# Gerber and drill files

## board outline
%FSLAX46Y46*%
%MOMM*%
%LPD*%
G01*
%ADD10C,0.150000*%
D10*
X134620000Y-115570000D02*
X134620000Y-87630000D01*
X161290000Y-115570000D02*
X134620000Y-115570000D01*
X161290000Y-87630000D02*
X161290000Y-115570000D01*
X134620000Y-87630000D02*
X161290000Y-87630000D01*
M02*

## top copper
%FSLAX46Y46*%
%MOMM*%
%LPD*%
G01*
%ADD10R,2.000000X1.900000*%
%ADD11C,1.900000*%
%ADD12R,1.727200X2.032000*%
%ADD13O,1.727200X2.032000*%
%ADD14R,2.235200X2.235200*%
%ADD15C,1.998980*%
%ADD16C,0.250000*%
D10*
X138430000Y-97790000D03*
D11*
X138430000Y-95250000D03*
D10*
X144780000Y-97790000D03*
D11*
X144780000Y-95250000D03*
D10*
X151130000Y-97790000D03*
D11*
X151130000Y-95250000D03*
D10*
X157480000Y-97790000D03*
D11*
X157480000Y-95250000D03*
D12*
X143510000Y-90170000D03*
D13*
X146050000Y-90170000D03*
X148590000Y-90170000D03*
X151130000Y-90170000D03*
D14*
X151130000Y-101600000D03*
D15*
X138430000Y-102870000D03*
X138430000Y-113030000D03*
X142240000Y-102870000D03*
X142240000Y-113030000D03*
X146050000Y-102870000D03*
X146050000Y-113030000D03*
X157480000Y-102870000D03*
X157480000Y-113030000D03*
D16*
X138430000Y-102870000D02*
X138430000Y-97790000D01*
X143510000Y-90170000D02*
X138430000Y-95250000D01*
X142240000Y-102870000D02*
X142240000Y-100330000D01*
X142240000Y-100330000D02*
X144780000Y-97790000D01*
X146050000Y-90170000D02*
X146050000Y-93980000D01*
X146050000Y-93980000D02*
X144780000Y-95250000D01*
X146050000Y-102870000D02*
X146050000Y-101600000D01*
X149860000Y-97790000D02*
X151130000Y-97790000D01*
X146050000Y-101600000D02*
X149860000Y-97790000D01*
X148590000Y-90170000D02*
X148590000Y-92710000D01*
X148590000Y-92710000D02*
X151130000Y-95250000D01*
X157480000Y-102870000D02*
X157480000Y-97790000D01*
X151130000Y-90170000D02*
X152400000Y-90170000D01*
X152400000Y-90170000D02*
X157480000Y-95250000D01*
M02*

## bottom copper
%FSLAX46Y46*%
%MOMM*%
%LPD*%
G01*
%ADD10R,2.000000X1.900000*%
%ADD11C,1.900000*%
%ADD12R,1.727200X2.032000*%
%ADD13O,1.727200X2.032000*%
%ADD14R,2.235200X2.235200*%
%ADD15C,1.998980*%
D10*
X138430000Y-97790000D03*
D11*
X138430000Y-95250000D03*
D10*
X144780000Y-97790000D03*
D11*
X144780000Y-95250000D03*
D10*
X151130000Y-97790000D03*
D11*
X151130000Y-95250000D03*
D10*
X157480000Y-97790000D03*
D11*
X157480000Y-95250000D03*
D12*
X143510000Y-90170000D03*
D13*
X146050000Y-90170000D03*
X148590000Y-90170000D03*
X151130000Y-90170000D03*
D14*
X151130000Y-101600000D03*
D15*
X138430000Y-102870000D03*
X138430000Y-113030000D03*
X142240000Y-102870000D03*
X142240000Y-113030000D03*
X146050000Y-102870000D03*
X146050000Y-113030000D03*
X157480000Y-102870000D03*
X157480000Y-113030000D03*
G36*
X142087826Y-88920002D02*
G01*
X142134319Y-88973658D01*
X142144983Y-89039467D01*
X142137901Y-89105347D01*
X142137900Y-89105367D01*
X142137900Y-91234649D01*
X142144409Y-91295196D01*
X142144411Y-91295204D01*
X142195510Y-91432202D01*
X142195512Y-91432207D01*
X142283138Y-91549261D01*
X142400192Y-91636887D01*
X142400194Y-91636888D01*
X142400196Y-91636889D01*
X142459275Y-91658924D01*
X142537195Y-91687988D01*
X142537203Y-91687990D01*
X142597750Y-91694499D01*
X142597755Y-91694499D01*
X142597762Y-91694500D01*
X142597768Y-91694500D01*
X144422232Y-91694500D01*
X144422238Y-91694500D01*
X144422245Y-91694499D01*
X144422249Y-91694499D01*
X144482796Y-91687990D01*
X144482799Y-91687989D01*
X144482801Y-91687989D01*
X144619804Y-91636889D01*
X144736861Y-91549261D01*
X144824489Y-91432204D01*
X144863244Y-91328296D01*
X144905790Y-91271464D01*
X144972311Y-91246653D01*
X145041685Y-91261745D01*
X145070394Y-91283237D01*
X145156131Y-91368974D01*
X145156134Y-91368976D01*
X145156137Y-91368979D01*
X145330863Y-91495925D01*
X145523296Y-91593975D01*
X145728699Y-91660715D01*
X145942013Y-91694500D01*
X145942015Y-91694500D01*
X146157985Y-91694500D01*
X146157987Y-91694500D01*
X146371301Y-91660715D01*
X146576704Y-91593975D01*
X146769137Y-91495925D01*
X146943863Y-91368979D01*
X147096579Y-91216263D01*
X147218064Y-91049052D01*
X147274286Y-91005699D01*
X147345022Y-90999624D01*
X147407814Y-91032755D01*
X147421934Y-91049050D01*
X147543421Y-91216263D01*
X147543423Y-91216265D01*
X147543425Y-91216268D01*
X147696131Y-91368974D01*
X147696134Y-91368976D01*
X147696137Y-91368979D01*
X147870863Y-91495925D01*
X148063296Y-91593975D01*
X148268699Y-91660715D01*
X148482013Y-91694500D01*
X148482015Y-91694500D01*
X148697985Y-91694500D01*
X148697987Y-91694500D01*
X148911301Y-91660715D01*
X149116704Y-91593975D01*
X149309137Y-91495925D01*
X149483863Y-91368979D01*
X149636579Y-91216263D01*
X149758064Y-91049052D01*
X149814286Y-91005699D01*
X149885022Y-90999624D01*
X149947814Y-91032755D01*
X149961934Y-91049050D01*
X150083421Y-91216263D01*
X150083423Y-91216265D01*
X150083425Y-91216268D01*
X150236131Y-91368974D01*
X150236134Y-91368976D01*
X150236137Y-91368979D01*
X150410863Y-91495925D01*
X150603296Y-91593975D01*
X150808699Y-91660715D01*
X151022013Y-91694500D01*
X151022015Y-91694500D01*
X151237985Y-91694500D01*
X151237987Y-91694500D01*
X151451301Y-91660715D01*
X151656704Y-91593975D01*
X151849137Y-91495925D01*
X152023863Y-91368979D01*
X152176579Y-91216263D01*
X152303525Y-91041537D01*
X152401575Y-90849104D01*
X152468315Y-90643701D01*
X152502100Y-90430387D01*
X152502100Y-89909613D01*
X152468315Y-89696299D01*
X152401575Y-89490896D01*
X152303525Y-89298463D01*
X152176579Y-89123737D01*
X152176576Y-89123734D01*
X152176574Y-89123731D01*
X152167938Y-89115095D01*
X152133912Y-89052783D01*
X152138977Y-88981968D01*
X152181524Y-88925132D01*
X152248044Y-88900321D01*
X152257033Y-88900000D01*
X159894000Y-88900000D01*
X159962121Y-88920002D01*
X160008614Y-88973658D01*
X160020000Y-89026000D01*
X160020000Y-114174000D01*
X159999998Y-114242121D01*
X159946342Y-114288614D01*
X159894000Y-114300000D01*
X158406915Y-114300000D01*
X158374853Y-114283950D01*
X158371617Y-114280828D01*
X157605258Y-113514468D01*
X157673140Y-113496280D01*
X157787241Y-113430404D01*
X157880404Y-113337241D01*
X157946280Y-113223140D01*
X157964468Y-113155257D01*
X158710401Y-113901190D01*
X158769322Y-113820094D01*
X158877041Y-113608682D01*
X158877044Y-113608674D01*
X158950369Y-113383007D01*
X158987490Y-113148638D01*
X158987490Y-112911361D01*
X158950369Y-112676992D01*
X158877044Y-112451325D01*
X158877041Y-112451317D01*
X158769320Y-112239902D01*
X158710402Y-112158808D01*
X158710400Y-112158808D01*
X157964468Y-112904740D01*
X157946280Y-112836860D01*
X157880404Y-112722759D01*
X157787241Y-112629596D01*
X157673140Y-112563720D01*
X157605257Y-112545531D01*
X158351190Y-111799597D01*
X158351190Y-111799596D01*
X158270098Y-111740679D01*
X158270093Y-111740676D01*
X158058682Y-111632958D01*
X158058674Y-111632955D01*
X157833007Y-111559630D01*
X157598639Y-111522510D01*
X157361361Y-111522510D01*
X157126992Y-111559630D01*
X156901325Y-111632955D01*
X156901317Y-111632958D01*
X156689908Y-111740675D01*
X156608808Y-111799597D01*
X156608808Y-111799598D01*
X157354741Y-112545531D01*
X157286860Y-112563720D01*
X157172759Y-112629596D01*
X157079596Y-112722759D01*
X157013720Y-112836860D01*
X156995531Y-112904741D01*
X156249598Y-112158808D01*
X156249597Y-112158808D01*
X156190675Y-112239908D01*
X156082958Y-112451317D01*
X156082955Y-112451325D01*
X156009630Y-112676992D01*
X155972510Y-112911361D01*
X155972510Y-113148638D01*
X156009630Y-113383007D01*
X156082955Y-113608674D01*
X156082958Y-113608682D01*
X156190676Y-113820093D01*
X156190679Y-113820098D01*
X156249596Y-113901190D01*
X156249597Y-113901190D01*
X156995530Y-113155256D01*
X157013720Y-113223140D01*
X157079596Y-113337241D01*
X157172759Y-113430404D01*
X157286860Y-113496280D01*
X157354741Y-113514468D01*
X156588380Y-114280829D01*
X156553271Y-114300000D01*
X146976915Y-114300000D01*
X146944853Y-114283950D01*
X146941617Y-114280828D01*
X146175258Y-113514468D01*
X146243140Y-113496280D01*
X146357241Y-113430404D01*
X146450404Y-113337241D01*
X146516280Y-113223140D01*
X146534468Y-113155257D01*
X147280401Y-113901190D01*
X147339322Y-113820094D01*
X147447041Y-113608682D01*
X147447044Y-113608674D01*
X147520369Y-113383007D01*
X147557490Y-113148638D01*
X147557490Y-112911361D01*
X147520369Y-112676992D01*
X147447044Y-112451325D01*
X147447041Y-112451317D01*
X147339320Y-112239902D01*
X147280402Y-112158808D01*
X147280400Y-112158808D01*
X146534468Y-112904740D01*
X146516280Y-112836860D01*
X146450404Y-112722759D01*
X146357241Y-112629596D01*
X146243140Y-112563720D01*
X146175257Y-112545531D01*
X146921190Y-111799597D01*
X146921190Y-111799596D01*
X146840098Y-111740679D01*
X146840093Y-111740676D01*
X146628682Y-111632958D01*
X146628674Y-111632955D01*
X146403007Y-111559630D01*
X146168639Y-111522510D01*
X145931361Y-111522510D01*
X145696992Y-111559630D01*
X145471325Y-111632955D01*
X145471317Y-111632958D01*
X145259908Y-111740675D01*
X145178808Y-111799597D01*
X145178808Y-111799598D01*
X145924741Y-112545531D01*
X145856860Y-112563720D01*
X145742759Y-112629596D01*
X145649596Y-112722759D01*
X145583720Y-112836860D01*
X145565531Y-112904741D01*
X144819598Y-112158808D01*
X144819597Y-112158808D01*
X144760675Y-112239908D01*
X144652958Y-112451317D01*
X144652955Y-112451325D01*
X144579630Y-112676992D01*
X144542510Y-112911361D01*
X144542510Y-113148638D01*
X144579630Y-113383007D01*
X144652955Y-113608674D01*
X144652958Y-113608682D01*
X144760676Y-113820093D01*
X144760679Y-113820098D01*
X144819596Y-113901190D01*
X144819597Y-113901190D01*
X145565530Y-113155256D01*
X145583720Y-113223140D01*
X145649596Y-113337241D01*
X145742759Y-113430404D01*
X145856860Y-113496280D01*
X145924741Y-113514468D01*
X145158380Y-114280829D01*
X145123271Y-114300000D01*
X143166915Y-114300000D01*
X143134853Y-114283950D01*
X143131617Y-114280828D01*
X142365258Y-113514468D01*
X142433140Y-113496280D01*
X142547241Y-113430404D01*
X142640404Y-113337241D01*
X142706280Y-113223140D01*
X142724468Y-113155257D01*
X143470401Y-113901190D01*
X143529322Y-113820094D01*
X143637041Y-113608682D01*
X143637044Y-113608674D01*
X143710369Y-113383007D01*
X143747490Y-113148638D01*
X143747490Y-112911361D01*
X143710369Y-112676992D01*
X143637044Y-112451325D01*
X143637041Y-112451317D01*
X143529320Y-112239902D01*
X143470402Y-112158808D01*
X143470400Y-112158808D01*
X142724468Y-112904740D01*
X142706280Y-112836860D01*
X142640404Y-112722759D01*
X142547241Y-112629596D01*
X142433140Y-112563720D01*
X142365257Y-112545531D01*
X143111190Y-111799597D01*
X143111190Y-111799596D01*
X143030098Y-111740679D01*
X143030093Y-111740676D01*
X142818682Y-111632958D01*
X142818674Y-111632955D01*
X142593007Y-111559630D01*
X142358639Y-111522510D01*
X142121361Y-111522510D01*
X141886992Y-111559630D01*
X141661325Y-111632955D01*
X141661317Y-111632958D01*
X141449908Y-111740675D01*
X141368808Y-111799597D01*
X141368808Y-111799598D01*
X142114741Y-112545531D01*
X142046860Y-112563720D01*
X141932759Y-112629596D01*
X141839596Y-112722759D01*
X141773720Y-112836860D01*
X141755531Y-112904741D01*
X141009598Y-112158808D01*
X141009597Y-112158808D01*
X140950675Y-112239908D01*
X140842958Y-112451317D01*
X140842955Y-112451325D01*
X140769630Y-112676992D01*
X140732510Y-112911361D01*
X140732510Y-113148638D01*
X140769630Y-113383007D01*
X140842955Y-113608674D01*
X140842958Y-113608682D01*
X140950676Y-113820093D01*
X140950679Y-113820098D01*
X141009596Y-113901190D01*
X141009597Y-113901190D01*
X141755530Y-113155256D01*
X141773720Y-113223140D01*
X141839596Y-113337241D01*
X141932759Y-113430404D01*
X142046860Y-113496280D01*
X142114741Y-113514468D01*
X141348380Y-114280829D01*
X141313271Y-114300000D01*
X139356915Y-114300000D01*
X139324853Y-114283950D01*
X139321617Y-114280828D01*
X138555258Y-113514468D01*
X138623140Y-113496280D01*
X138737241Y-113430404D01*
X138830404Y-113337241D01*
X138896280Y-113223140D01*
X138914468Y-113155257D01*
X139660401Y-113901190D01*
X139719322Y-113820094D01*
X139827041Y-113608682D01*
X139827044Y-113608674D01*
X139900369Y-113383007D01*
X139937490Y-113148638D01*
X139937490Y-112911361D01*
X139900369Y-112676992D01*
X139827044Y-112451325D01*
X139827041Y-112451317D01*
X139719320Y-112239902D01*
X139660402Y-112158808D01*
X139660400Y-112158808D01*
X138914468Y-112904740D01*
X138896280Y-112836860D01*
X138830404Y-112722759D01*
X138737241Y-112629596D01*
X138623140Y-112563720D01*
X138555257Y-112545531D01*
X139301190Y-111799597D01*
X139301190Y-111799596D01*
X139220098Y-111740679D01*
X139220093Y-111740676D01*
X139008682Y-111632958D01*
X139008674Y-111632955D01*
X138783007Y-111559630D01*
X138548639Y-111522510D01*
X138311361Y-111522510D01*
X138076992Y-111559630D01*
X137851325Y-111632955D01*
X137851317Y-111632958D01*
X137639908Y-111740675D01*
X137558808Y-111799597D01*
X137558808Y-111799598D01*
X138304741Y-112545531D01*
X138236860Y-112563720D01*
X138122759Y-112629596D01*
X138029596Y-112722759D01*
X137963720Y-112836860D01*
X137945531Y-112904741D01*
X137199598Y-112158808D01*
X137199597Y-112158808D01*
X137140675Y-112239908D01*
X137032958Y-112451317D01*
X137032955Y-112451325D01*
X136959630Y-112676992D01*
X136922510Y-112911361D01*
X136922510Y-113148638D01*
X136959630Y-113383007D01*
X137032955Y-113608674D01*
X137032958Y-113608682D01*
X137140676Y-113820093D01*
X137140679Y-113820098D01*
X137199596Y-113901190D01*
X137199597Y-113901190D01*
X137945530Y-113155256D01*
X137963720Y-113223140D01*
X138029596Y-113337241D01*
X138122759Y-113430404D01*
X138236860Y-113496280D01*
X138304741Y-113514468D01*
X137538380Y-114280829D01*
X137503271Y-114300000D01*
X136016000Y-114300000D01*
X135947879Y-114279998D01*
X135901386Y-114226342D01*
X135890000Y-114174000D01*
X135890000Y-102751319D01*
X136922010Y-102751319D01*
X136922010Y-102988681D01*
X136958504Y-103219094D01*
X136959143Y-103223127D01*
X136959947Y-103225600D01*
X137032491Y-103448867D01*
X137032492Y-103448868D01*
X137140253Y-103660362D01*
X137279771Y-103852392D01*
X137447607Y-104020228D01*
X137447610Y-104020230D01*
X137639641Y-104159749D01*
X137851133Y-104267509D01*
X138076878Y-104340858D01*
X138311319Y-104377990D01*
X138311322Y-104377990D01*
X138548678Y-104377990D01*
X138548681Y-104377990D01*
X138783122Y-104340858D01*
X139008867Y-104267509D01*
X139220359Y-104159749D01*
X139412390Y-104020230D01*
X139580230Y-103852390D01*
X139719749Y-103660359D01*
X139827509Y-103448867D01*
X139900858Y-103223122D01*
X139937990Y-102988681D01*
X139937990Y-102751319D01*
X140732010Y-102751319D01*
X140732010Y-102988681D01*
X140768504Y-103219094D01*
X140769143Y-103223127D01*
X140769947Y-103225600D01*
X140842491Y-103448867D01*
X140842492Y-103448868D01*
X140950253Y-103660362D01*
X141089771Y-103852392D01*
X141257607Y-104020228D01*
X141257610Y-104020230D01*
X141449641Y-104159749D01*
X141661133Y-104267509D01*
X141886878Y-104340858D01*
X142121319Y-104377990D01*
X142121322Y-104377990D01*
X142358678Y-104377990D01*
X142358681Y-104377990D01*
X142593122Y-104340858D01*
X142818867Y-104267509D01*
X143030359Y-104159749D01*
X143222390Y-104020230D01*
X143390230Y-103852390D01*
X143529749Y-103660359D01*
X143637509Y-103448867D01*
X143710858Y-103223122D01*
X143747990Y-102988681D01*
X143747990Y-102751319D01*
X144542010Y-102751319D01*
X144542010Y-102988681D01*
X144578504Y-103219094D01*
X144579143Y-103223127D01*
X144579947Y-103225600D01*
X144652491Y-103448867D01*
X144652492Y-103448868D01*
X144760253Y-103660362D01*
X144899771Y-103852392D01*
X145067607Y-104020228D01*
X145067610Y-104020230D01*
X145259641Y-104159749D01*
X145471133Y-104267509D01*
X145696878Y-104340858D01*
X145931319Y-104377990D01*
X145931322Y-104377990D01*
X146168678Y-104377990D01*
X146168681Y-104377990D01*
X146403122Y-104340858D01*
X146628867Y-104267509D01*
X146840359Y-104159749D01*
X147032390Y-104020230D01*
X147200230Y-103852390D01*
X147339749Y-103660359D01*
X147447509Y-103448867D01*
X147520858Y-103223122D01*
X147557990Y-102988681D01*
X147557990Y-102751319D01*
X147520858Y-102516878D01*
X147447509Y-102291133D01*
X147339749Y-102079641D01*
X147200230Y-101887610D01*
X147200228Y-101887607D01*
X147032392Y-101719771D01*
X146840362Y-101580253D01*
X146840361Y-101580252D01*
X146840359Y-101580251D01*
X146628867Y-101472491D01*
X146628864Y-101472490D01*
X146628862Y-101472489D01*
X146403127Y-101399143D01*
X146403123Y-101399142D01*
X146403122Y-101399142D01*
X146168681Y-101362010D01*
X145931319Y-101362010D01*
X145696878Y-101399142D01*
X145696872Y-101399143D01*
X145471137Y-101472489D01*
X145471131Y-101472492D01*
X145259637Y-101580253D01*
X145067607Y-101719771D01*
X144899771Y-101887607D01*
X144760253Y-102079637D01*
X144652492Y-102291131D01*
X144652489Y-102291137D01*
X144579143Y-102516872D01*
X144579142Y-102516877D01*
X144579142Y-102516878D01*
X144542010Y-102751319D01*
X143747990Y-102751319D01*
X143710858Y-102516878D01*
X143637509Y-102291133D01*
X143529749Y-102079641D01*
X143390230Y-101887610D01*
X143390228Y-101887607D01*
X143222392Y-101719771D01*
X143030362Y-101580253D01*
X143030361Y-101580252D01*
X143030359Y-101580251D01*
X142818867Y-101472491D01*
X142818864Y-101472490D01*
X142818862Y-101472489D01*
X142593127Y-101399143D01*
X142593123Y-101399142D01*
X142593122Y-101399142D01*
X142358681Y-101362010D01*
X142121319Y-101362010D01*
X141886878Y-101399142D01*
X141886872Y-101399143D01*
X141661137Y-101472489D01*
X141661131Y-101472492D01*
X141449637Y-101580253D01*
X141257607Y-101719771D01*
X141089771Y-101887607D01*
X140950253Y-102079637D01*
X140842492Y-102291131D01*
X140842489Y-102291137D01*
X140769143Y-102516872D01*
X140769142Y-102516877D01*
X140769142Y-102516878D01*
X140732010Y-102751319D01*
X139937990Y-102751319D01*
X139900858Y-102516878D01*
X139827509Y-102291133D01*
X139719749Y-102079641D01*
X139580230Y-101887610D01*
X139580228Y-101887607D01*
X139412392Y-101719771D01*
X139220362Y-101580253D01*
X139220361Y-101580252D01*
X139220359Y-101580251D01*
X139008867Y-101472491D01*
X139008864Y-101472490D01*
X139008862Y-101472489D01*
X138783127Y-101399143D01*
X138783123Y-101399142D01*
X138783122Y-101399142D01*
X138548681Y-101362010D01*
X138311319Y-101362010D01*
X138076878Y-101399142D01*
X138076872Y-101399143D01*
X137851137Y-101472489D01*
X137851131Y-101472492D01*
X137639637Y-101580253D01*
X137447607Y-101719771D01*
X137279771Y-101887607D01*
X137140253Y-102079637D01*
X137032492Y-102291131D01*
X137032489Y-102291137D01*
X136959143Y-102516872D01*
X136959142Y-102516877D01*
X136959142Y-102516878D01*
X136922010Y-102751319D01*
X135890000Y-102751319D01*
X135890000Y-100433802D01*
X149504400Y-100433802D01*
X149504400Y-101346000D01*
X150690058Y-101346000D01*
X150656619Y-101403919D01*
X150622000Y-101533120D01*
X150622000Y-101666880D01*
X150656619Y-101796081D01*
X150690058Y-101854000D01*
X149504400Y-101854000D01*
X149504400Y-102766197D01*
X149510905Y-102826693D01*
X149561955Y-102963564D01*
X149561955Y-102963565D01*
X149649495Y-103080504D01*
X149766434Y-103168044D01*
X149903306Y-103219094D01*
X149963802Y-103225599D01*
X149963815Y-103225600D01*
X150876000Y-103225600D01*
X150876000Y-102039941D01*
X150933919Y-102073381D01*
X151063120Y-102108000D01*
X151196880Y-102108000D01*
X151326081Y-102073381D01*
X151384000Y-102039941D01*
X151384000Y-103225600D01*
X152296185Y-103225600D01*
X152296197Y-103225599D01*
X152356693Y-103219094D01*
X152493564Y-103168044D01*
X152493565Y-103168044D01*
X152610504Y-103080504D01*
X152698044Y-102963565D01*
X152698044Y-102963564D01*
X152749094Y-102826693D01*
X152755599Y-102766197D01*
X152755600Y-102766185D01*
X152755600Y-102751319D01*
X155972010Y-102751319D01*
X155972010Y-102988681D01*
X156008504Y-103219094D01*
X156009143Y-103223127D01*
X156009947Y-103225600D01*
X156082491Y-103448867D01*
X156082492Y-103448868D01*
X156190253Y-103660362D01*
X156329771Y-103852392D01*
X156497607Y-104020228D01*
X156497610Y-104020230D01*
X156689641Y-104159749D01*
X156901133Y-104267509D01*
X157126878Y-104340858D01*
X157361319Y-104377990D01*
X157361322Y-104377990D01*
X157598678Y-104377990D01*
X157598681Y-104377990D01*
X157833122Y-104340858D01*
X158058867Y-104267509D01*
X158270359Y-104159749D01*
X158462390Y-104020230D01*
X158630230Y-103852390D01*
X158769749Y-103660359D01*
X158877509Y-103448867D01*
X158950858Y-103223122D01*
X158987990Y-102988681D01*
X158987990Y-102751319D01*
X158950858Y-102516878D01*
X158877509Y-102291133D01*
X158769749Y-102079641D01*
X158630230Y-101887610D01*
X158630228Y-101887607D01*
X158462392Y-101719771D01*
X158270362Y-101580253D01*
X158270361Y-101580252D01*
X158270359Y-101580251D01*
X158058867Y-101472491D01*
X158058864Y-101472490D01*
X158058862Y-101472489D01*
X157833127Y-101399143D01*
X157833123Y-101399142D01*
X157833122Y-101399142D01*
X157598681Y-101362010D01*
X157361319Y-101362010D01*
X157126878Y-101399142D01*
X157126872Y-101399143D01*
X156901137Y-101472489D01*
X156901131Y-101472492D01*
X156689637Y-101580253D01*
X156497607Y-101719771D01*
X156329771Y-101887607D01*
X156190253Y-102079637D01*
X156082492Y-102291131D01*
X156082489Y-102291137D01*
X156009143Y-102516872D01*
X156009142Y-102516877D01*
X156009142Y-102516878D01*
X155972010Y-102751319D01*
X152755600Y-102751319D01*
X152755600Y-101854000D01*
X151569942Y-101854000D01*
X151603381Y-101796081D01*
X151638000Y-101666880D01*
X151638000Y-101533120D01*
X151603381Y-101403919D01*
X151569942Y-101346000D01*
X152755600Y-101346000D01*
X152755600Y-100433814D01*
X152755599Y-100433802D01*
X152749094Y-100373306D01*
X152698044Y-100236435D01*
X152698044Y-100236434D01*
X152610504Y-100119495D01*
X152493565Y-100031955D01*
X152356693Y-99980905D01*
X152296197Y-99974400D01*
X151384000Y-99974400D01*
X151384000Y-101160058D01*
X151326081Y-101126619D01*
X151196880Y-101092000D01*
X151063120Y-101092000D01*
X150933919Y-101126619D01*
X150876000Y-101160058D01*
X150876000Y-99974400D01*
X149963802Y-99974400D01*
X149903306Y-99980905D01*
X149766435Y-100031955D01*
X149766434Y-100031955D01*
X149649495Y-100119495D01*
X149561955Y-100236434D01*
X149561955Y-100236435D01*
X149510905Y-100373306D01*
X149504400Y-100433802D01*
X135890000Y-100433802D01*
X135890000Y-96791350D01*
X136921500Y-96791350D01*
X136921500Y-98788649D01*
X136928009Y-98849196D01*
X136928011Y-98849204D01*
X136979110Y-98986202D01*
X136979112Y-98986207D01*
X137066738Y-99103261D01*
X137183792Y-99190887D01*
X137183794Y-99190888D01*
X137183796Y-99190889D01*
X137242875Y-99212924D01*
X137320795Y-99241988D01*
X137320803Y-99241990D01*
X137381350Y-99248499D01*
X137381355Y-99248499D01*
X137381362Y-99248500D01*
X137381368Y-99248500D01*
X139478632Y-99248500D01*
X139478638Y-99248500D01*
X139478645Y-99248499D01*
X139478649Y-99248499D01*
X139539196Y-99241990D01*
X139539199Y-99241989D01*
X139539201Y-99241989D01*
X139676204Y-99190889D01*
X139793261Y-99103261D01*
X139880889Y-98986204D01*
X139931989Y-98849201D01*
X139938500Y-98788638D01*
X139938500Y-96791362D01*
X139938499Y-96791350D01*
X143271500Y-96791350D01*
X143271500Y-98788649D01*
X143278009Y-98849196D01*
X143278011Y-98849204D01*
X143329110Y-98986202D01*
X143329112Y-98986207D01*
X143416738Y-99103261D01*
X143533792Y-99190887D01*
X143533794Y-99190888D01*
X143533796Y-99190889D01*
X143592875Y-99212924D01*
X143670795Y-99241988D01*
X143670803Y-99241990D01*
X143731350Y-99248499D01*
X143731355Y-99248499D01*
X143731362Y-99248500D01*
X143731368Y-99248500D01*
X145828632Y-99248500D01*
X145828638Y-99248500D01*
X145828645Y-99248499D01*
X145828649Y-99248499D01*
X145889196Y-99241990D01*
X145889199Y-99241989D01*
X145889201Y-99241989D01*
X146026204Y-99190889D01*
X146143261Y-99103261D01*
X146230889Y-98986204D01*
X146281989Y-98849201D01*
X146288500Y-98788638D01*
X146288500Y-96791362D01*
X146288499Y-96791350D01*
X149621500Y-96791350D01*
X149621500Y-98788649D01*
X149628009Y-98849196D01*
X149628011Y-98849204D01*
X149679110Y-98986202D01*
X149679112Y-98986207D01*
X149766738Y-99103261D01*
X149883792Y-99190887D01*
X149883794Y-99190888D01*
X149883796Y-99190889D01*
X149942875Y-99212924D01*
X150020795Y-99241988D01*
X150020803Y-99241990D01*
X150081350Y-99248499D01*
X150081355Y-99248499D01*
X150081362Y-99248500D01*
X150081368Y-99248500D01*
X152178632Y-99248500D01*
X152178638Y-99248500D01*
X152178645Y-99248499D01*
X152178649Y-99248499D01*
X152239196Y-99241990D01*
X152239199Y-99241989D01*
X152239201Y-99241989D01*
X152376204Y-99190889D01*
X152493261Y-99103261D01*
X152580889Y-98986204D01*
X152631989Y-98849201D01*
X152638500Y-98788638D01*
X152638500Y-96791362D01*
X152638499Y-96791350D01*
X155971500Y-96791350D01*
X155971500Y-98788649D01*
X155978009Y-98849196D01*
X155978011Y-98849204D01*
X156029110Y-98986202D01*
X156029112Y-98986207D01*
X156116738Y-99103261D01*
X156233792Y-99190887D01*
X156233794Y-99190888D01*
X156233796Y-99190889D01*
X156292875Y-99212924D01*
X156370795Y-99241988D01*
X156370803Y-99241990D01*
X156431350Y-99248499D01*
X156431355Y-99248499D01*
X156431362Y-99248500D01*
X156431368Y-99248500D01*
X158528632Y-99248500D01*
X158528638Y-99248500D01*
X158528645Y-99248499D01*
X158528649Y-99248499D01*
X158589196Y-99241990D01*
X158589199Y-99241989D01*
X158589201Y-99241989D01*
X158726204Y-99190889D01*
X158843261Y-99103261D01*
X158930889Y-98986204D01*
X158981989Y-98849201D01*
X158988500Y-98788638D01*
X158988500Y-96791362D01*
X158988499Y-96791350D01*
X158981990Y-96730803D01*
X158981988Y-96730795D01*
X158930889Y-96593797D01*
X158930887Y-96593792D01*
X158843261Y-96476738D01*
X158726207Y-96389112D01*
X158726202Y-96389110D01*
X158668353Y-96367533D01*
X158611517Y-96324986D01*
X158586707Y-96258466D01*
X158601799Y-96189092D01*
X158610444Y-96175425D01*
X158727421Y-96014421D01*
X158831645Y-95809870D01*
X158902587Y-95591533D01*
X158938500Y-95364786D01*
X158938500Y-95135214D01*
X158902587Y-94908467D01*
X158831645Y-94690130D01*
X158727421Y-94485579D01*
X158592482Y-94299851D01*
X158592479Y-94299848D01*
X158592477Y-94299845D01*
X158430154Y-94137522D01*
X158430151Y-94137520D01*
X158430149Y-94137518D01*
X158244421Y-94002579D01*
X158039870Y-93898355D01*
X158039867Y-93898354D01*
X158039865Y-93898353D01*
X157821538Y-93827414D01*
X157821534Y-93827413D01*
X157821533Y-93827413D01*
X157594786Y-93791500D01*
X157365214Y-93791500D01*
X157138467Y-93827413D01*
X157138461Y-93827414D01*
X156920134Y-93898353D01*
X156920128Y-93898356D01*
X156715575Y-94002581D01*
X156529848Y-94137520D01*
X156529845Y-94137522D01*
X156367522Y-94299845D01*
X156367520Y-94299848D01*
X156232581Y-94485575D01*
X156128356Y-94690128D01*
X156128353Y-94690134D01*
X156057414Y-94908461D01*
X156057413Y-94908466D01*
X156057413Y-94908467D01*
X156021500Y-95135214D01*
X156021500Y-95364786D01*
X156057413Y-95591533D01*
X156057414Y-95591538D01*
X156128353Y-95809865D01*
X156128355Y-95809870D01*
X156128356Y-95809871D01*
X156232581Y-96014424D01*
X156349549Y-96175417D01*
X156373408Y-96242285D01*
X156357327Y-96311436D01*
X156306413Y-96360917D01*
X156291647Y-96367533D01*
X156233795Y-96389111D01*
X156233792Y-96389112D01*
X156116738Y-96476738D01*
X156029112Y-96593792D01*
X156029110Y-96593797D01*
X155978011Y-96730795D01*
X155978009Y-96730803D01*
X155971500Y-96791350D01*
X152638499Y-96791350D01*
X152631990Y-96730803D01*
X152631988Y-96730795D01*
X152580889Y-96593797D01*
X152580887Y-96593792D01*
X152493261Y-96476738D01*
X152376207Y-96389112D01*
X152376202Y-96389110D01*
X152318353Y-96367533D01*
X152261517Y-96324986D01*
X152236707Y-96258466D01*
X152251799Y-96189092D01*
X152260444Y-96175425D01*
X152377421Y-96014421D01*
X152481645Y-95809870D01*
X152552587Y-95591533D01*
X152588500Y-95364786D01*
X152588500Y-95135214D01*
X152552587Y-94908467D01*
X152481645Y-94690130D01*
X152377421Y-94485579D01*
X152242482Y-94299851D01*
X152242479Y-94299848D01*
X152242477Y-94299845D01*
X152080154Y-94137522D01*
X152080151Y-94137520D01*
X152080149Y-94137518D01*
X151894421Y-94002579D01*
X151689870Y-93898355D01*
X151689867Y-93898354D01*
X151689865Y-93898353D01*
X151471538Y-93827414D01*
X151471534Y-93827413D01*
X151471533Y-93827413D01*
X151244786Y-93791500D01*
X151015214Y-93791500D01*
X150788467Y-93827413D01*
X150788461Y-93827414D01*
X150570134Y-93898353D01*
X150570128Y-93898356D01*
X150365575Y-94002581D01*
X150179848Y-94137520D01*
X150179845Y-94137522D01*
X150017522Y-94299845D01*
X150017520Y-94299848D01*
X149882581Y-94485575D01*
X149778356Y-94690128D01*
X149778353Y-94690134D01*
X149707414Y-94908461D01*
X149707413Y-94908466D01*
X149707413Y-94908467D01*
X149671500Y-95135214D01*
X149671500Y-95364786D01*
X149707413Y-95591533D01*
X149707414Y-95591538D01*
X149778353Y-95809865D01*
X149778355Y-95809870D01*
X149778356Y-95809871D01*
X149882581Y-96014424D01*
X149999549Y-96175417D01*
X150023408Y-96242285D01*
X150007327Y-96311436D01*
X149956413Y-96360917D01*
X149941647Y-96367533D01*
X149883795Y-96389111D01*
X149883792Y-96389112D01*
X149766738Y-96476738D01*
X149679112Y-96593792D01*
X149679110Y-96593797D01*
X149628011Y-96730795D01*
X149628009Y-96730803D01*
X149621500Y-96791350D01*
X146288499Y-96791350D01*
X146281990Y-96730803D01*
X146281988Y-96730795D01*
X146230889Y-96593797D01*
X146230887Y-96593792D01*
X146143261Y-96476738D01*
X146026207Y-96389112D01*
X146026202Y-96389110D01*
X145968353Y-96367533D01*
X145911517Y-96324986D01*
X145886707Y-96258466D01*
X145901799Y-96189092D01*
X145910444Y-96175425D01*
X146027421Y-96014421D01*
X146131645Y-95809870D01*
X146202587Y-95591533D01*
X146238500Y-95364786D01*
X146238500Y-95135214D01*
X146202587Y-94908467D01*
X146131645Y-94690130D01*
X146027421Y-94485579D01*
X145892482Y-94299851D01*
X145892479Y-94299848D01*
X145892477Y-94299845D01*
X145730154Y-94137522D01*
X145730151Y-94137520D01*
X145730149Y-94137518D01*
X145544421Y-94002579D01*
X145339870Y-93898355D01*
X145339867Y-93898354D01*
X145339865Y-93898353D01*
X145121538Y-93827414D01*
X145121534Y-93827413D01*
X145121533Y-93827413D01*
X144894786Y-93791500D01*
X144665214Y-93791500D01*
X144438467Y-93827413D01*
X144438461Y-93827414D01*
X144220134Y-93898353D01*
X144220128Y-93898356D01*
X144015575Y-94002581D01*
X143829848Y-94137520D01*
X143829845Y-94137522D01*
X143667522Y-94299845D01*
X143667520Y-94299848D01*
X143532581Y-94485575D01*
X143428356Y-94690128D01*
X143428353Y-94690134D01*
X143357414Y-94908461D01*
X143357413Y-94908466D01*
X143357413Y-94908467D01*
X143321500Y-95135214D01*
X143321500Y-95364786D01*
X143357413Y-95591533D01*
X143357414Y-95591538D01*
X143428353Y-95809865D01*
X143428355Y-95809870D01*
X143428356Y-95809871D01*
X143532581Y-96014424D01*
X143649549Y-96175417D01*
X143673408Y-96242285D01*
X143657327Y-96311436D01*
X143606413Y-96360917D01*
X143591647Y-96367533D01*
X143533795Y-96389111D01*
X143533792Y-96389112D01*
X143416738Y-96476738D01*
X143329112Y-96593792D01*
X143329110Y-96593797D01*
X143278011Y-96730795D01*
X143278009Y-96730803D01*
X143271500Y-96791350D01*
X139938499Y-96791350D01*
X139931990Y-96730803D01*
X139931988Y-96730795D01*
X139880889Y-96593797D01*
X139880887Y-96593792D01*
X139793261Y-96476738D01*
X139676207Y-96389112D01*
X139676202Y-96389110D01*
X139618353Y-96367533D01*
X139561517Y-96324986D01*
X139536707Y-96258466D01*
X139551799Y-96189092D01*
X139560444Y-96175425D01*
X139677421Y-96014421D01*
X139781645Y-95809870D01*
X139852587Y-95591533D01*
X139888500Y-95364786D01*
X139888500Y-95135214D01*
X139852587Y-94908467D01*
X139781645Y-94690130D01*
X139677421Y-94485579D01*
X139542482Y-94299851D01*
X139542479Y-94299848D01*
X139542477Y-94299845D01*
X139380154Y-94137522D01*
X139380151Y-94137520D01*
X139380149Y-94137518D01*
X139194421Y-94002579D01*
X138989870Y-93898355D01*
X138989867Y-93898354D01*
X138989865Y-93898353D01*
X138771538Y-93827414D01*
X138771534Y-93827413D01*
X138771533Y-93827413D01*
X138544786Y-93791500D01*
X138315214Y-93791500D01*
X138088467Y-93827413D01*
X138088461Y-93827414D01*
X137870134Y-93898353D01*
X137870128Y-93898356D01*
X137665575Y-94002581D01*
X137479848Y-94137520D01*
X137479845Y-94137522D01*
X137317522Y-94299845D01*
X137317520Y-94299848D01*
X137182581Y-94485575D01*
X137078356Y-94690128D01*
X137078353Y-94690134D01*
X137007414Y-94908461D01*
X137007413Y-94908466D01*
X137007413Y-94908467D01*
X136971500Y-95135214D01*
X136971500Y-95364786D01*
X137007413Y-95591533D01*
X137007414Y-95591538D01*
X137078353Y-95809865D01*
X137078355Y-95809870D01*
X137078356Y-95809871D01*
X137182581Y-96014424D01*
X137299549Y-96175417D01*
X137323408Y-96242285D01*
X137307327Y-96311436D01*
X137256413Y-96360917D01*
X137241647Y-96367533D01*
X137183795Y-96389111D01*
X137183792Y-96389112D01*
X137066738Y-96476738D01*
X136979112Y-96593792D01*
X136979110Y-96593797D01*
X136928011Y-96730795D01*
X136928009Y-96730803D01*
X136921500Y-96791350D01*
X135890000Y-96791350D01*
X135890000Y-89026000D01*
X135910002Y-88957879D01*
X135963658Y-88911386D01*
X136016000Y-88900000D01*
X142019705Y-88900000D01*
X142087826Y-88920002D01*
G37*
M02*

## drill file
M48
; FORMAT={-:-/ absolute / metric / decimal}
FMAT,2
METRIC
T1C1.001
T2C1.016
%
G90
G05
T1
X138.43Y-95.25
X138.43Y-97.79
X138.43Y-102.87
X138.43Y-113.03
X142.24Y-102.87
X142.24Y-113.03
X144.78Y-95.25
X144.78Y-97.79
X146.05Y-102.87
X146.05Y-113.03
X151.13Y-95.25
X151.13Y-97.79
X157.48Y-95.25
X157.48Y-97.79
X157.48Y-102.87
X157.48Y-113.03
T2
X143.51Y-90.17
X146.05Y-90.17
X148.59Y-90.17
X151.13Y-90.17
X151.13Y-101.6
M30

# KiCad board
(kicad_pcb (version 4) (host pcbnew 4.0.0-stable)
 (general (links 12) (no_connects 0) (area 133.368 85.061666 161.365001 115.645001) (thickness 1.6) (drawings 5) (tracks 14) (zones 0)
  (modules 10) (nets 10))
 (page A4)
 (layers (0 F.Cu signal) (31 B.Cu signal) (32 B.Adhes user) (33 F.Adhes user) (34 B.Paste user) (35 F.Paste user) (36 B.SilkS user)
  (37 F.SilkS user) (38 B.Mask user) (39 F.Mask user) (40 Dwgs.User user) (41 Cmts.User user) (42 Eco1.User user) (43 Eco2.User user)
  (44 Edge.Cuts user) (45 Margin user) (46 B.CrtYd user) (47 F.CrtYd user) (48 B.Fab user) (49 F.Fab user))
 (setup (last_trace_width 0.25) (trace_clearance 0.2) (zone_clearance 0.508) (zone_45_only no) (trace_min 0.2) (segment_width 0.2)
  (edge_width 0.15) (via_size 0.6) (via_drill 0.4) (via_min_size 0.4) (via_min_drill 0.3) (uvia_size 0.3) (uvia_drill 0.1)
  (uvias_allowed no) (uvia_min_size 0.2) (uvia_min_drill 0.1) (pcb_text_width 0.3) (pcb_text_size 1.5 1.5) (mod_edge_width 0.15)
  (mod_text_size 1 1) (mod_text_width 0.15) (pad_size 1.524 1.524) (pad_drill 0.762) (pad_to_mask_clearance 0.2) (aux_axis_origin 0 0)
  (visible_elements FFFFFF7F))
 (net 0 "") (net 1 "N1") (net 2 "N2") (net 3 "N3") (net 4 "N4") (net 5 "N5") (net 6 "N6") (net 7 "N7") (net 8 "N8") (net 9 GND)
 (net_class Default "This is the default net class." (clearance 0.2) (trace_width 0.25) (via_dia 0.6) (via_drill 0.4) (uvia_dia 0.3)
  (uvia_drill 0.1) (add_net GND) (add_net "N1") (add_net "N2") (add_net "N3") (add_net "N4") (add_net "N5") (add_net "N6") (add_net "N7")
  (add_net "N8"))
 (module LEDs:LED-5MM (layer F.Cu) (at 138.43 97.79 90)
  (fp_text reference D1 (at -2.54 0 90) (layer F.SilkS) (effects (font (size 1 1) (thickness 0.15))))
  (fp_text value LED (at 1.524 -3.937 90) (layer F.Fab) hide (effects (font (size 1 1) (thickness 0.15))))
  (pad 1 thru_hole rect (at 0 0 180) (size 2 1.9) (drill 1.00076) (layers *.Cu *.Mask F.SilkS) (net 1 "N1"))
  (pad 2 thru_hole circle (at 2.54 0 90) (size 1.9 1.9) (drill 1.00076) (layers *.Cu *.Mask F.SilkS) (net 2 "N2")))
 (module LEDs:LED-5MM (layer F.Cu) (at 144.78 97.79 90)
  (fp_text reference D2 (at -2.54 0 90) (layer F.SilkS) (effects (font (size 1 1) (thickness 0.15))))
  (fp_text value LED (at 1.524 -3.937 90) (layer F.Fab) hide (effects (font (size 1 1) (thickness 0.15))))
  (pad 1 thru_hole rect (at 0 0 180) (size 2 1.9) (drill 1.00076) (layers *.Cu *.Mask F.SilkS) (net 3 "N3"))
  (pad 2 thru_hole circle (at 2.54 0 90) (size 1.9 1.9) (drill 1.00076) (layers *.Cu *.Mask F.SilkS) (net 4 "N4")))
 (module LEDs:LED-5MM (layer F.Cu) (at 151.13 97.79 90)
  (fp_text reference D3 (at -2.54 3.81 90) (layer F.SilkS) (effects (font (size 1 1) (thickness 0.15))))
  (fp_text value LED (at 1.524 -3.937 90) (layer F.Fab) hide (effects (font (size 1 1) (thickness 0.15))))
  (pad 1 thru_hole rect (at 0 0 180) (size 2 1.9) (drill 1.00076) (layers *.Cu *.Mask F.SilkS) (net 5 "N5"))
  (pad 2 thru_hole circle (at 2.54 0 90) (size 1.9 1.9) (drill 1.00076) (layers *.Cu *.Mask F.SilkS) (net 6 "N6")))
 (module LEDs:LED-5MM (layer F.Cu) (at 157.48 97.79 90)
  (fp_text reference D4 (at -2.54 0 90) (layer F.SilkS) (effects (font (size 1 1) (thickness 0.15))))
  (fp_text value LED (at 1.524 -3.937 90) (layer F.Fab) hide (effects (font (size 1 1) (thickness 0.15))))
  (pad 1 thru_hole rect (at 0 0 180) (size 2 1.9) (drill 1.00076) (layers *.Cu *.Mask F.SilkS) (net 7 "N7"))
  (pad 2 thru_hole circle (at 2.54 0 90) (size 1.9 1.9) (drill 1.00076) (layers *.Cu *.Mask F.SilkS) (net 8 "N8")))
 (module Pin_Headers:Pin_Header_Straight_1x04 (layer F.Cu) (at 143.51 90.17 90)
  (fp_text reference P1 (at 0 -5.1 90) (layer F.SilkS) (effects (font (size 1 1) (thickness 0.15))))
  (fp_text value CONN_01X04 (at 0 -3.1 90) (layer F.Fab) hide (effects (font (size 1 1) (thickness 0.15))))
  (pad 1 thru_hole rect (at 0 0 90) (size 2.032 1.7272) (drill 1.016) (layers *.Cu *.Mask F.SilkS) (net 2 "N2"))
  (pad 2 thru_hole oval (at 0 2.54 90) (size 2.032 1.7272) (drill 1.016) (layers *.Cu *.Mask F.SilkS) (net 4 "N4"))
  (pad 3 thru_hole oval (at 0 5.08 90) (size 2.032 1.7272) (drill 1.016) (layers *.Cu *.Mask F.SilkS) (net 6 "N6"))
  (pad 4 thru_hole oval (at 0 7.62 90) (size 2.032 1.7272) (drill 1.016) (layers *.Cu *.Mask F.SilkS) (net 8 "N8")))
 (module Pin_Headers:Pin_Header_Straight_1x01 (layer F.Cu) (at 151.13 101.6)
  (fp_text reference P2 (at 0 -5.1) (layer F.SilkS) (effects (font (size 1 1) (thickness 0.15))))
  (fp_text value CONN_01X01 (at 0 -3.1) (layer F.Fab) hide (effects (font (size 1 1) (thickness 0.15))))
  (pad 1 thru_hole rect (at 0 0) (size 2.2352 2.2352) (drill 1.016) (layers *.Cu *.Mask F.SilkS) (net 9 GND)))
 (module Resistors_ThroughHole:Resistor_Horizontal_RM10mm (layer F.Cu) (at 138.43 107.95 270)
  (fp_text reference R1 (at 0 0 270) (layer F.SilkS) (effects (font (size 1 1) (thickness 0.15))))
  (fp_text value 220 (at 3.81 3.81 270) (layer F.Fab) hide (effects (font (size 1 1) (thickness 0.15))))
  (pad 1 thru_hole circle (at -5.08 0 270) (size 1.99898 1.99898) (drill 1.00076) (layers *.Cu *.SilkS *.Mask) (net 1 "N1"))
  (pad 2 thru_hole circle (at 5.08 0 270) (size 1.99898 1.99898) (drill 1.00076) (layers *.Cu *.SilkS *.Mask) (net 9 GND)))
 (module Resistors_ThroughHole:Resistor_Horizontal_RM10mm (layer F.Cu) (at 142.24 107.95 270)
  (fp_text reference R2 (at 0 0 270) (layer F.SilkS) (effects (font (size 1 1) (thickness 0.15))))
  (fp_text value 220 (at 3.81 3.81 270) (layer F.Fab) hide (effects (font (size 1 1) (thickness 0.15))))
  (pad 1 thru_hole circle (at -5.08 0 270) (size 1.99898 1.99898) (drill 1.00076) (layers *.Cu *.SilkS *.Mask) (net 3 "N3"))
  (pad 2 thru_hole circle (at 5.08 0 270) (size 1.99898 1.99898) (drill 1.00076) (layers *.Cu *.SilkS *.Mask) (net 9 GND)))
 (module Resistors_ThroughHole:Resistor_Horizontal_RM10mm (layer F.Cu) (at 146.05 107.95 270)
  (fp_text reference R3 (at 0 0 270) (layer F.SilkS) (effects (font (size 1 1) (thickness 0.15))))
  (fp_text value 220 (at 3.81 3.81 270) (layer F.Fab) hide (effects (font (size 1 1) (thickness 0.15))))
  (pad 1 thru_hole circle (at -5.08 0 270) (size 1.99898 1.99898) (drill 1.00076) (layers *.Cu *.SilkS *.Mask) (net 5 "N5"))
  (pad 2 thru_hole circle (at 5.08 0 270) (size 1.99898 1.99898) (drill 1.00076) (layers *.Cu *.SilkS *.Mask) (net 9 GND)))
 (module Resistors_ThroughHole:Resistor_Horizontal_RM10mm (layer F.Cu) (at 157.48 107.95 270)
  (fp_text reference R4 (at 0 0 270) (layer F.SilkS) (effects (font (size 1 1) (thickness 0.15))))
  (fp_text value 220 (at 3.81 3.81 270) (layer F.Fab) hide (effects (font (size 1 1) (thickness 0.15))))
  (pad 1 thru_hole circle (at -5.08 0 270) (size 1.99898 1.99898) (drill 1.00076) (layers *.Cu *.SilkS *.Mask) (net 7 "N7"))
  (pad 2 thru_hole circle (at 5.08 0 270) (size 1.99898 1.99898) (drill 1.00076) (layers *.Cu *.SilkS *.Mask) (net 9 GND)))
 (gr_line (start 134.62 115.57) (end 134.62 87.63) (angle 90) (layer Edge.Cuts) (width 0.15))
 (gr_line (start 161.29 115.57) (end 134.62 115.57) (angle 90) (layer Edge.Cuts) (width 0.15))
 (gr_line (start 161.29 87.63) (end 161.29 115.57) (angle 90) (layer Edge.Cuts) (width 0.15))
 (gr_line (start 134.62 87.63) (end 161.29 87.63) (angle 90) (layer Edge.Cuts) (width 0.15))
 (segment (start 138.43 102.87) (end 138.43 97.79) (width 0.25) (layer F.Cu) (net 1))
 (segment (start 143.51 90.17) (end 138.43 95.25) (width 0.25) (layer F.Cu) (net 2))
 (segment (start 142.24 102.87) (end 142.24 100.33) (width 0.25) (layer F.Cu) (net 3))
 (segment (start 142.24 100.33) (end 144.78 97.79) (width 0.25) (layer F.Cu) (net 3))
 (segment (start 146.05 90.17) (end 146.05 93.98) (width 0.25) (layer F.Cu) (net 4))
 (segment (start 146.05 93.98) (end 144.78 95.25) (width 0.25) (layer F.Cu) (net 4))
 (segment (start 146.05 102.87) (end 146.05 101.6) (width 0.25) (layer F.Cu) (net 5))
 (segment (start 149.86 97.79) (end 151.13 97.79) (width 0.25) (layer F.Cu) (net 5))
 (segment (start 146.05 101.6) (end 149.86 97.79) (width 0.25) (layer F.Cu) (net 5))
 (segment (start 148.59 90.17) (end 148.59 92.71) (width 0.25) (layer F.Cu) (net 6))
 (segment (start 148.59 92.71) (end 151.13 95.25) (width 0.25) (layer F.Cu) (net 6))
 (segment (start 157.48 102.87) (end 157.48 97.79) (width 0.25) (layer F.Cu) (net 7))
 (segment (start 151.13 90.17) (end 152.4 90.17) (width 0.25) (layer F.Cu) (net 8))
 (segment (start 152.4 90.17) (end 157.48 95.25) (width 0.25) (layer F.Cu) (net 8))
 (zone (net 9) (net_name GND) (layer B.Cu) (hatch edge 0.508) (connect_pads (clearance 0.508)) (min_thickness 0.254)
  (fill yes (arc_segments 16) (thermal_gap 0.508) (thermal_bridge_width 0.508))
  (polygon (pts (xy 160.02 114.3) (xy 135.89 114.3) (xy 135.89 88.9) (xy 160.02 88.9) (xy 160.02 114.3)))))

